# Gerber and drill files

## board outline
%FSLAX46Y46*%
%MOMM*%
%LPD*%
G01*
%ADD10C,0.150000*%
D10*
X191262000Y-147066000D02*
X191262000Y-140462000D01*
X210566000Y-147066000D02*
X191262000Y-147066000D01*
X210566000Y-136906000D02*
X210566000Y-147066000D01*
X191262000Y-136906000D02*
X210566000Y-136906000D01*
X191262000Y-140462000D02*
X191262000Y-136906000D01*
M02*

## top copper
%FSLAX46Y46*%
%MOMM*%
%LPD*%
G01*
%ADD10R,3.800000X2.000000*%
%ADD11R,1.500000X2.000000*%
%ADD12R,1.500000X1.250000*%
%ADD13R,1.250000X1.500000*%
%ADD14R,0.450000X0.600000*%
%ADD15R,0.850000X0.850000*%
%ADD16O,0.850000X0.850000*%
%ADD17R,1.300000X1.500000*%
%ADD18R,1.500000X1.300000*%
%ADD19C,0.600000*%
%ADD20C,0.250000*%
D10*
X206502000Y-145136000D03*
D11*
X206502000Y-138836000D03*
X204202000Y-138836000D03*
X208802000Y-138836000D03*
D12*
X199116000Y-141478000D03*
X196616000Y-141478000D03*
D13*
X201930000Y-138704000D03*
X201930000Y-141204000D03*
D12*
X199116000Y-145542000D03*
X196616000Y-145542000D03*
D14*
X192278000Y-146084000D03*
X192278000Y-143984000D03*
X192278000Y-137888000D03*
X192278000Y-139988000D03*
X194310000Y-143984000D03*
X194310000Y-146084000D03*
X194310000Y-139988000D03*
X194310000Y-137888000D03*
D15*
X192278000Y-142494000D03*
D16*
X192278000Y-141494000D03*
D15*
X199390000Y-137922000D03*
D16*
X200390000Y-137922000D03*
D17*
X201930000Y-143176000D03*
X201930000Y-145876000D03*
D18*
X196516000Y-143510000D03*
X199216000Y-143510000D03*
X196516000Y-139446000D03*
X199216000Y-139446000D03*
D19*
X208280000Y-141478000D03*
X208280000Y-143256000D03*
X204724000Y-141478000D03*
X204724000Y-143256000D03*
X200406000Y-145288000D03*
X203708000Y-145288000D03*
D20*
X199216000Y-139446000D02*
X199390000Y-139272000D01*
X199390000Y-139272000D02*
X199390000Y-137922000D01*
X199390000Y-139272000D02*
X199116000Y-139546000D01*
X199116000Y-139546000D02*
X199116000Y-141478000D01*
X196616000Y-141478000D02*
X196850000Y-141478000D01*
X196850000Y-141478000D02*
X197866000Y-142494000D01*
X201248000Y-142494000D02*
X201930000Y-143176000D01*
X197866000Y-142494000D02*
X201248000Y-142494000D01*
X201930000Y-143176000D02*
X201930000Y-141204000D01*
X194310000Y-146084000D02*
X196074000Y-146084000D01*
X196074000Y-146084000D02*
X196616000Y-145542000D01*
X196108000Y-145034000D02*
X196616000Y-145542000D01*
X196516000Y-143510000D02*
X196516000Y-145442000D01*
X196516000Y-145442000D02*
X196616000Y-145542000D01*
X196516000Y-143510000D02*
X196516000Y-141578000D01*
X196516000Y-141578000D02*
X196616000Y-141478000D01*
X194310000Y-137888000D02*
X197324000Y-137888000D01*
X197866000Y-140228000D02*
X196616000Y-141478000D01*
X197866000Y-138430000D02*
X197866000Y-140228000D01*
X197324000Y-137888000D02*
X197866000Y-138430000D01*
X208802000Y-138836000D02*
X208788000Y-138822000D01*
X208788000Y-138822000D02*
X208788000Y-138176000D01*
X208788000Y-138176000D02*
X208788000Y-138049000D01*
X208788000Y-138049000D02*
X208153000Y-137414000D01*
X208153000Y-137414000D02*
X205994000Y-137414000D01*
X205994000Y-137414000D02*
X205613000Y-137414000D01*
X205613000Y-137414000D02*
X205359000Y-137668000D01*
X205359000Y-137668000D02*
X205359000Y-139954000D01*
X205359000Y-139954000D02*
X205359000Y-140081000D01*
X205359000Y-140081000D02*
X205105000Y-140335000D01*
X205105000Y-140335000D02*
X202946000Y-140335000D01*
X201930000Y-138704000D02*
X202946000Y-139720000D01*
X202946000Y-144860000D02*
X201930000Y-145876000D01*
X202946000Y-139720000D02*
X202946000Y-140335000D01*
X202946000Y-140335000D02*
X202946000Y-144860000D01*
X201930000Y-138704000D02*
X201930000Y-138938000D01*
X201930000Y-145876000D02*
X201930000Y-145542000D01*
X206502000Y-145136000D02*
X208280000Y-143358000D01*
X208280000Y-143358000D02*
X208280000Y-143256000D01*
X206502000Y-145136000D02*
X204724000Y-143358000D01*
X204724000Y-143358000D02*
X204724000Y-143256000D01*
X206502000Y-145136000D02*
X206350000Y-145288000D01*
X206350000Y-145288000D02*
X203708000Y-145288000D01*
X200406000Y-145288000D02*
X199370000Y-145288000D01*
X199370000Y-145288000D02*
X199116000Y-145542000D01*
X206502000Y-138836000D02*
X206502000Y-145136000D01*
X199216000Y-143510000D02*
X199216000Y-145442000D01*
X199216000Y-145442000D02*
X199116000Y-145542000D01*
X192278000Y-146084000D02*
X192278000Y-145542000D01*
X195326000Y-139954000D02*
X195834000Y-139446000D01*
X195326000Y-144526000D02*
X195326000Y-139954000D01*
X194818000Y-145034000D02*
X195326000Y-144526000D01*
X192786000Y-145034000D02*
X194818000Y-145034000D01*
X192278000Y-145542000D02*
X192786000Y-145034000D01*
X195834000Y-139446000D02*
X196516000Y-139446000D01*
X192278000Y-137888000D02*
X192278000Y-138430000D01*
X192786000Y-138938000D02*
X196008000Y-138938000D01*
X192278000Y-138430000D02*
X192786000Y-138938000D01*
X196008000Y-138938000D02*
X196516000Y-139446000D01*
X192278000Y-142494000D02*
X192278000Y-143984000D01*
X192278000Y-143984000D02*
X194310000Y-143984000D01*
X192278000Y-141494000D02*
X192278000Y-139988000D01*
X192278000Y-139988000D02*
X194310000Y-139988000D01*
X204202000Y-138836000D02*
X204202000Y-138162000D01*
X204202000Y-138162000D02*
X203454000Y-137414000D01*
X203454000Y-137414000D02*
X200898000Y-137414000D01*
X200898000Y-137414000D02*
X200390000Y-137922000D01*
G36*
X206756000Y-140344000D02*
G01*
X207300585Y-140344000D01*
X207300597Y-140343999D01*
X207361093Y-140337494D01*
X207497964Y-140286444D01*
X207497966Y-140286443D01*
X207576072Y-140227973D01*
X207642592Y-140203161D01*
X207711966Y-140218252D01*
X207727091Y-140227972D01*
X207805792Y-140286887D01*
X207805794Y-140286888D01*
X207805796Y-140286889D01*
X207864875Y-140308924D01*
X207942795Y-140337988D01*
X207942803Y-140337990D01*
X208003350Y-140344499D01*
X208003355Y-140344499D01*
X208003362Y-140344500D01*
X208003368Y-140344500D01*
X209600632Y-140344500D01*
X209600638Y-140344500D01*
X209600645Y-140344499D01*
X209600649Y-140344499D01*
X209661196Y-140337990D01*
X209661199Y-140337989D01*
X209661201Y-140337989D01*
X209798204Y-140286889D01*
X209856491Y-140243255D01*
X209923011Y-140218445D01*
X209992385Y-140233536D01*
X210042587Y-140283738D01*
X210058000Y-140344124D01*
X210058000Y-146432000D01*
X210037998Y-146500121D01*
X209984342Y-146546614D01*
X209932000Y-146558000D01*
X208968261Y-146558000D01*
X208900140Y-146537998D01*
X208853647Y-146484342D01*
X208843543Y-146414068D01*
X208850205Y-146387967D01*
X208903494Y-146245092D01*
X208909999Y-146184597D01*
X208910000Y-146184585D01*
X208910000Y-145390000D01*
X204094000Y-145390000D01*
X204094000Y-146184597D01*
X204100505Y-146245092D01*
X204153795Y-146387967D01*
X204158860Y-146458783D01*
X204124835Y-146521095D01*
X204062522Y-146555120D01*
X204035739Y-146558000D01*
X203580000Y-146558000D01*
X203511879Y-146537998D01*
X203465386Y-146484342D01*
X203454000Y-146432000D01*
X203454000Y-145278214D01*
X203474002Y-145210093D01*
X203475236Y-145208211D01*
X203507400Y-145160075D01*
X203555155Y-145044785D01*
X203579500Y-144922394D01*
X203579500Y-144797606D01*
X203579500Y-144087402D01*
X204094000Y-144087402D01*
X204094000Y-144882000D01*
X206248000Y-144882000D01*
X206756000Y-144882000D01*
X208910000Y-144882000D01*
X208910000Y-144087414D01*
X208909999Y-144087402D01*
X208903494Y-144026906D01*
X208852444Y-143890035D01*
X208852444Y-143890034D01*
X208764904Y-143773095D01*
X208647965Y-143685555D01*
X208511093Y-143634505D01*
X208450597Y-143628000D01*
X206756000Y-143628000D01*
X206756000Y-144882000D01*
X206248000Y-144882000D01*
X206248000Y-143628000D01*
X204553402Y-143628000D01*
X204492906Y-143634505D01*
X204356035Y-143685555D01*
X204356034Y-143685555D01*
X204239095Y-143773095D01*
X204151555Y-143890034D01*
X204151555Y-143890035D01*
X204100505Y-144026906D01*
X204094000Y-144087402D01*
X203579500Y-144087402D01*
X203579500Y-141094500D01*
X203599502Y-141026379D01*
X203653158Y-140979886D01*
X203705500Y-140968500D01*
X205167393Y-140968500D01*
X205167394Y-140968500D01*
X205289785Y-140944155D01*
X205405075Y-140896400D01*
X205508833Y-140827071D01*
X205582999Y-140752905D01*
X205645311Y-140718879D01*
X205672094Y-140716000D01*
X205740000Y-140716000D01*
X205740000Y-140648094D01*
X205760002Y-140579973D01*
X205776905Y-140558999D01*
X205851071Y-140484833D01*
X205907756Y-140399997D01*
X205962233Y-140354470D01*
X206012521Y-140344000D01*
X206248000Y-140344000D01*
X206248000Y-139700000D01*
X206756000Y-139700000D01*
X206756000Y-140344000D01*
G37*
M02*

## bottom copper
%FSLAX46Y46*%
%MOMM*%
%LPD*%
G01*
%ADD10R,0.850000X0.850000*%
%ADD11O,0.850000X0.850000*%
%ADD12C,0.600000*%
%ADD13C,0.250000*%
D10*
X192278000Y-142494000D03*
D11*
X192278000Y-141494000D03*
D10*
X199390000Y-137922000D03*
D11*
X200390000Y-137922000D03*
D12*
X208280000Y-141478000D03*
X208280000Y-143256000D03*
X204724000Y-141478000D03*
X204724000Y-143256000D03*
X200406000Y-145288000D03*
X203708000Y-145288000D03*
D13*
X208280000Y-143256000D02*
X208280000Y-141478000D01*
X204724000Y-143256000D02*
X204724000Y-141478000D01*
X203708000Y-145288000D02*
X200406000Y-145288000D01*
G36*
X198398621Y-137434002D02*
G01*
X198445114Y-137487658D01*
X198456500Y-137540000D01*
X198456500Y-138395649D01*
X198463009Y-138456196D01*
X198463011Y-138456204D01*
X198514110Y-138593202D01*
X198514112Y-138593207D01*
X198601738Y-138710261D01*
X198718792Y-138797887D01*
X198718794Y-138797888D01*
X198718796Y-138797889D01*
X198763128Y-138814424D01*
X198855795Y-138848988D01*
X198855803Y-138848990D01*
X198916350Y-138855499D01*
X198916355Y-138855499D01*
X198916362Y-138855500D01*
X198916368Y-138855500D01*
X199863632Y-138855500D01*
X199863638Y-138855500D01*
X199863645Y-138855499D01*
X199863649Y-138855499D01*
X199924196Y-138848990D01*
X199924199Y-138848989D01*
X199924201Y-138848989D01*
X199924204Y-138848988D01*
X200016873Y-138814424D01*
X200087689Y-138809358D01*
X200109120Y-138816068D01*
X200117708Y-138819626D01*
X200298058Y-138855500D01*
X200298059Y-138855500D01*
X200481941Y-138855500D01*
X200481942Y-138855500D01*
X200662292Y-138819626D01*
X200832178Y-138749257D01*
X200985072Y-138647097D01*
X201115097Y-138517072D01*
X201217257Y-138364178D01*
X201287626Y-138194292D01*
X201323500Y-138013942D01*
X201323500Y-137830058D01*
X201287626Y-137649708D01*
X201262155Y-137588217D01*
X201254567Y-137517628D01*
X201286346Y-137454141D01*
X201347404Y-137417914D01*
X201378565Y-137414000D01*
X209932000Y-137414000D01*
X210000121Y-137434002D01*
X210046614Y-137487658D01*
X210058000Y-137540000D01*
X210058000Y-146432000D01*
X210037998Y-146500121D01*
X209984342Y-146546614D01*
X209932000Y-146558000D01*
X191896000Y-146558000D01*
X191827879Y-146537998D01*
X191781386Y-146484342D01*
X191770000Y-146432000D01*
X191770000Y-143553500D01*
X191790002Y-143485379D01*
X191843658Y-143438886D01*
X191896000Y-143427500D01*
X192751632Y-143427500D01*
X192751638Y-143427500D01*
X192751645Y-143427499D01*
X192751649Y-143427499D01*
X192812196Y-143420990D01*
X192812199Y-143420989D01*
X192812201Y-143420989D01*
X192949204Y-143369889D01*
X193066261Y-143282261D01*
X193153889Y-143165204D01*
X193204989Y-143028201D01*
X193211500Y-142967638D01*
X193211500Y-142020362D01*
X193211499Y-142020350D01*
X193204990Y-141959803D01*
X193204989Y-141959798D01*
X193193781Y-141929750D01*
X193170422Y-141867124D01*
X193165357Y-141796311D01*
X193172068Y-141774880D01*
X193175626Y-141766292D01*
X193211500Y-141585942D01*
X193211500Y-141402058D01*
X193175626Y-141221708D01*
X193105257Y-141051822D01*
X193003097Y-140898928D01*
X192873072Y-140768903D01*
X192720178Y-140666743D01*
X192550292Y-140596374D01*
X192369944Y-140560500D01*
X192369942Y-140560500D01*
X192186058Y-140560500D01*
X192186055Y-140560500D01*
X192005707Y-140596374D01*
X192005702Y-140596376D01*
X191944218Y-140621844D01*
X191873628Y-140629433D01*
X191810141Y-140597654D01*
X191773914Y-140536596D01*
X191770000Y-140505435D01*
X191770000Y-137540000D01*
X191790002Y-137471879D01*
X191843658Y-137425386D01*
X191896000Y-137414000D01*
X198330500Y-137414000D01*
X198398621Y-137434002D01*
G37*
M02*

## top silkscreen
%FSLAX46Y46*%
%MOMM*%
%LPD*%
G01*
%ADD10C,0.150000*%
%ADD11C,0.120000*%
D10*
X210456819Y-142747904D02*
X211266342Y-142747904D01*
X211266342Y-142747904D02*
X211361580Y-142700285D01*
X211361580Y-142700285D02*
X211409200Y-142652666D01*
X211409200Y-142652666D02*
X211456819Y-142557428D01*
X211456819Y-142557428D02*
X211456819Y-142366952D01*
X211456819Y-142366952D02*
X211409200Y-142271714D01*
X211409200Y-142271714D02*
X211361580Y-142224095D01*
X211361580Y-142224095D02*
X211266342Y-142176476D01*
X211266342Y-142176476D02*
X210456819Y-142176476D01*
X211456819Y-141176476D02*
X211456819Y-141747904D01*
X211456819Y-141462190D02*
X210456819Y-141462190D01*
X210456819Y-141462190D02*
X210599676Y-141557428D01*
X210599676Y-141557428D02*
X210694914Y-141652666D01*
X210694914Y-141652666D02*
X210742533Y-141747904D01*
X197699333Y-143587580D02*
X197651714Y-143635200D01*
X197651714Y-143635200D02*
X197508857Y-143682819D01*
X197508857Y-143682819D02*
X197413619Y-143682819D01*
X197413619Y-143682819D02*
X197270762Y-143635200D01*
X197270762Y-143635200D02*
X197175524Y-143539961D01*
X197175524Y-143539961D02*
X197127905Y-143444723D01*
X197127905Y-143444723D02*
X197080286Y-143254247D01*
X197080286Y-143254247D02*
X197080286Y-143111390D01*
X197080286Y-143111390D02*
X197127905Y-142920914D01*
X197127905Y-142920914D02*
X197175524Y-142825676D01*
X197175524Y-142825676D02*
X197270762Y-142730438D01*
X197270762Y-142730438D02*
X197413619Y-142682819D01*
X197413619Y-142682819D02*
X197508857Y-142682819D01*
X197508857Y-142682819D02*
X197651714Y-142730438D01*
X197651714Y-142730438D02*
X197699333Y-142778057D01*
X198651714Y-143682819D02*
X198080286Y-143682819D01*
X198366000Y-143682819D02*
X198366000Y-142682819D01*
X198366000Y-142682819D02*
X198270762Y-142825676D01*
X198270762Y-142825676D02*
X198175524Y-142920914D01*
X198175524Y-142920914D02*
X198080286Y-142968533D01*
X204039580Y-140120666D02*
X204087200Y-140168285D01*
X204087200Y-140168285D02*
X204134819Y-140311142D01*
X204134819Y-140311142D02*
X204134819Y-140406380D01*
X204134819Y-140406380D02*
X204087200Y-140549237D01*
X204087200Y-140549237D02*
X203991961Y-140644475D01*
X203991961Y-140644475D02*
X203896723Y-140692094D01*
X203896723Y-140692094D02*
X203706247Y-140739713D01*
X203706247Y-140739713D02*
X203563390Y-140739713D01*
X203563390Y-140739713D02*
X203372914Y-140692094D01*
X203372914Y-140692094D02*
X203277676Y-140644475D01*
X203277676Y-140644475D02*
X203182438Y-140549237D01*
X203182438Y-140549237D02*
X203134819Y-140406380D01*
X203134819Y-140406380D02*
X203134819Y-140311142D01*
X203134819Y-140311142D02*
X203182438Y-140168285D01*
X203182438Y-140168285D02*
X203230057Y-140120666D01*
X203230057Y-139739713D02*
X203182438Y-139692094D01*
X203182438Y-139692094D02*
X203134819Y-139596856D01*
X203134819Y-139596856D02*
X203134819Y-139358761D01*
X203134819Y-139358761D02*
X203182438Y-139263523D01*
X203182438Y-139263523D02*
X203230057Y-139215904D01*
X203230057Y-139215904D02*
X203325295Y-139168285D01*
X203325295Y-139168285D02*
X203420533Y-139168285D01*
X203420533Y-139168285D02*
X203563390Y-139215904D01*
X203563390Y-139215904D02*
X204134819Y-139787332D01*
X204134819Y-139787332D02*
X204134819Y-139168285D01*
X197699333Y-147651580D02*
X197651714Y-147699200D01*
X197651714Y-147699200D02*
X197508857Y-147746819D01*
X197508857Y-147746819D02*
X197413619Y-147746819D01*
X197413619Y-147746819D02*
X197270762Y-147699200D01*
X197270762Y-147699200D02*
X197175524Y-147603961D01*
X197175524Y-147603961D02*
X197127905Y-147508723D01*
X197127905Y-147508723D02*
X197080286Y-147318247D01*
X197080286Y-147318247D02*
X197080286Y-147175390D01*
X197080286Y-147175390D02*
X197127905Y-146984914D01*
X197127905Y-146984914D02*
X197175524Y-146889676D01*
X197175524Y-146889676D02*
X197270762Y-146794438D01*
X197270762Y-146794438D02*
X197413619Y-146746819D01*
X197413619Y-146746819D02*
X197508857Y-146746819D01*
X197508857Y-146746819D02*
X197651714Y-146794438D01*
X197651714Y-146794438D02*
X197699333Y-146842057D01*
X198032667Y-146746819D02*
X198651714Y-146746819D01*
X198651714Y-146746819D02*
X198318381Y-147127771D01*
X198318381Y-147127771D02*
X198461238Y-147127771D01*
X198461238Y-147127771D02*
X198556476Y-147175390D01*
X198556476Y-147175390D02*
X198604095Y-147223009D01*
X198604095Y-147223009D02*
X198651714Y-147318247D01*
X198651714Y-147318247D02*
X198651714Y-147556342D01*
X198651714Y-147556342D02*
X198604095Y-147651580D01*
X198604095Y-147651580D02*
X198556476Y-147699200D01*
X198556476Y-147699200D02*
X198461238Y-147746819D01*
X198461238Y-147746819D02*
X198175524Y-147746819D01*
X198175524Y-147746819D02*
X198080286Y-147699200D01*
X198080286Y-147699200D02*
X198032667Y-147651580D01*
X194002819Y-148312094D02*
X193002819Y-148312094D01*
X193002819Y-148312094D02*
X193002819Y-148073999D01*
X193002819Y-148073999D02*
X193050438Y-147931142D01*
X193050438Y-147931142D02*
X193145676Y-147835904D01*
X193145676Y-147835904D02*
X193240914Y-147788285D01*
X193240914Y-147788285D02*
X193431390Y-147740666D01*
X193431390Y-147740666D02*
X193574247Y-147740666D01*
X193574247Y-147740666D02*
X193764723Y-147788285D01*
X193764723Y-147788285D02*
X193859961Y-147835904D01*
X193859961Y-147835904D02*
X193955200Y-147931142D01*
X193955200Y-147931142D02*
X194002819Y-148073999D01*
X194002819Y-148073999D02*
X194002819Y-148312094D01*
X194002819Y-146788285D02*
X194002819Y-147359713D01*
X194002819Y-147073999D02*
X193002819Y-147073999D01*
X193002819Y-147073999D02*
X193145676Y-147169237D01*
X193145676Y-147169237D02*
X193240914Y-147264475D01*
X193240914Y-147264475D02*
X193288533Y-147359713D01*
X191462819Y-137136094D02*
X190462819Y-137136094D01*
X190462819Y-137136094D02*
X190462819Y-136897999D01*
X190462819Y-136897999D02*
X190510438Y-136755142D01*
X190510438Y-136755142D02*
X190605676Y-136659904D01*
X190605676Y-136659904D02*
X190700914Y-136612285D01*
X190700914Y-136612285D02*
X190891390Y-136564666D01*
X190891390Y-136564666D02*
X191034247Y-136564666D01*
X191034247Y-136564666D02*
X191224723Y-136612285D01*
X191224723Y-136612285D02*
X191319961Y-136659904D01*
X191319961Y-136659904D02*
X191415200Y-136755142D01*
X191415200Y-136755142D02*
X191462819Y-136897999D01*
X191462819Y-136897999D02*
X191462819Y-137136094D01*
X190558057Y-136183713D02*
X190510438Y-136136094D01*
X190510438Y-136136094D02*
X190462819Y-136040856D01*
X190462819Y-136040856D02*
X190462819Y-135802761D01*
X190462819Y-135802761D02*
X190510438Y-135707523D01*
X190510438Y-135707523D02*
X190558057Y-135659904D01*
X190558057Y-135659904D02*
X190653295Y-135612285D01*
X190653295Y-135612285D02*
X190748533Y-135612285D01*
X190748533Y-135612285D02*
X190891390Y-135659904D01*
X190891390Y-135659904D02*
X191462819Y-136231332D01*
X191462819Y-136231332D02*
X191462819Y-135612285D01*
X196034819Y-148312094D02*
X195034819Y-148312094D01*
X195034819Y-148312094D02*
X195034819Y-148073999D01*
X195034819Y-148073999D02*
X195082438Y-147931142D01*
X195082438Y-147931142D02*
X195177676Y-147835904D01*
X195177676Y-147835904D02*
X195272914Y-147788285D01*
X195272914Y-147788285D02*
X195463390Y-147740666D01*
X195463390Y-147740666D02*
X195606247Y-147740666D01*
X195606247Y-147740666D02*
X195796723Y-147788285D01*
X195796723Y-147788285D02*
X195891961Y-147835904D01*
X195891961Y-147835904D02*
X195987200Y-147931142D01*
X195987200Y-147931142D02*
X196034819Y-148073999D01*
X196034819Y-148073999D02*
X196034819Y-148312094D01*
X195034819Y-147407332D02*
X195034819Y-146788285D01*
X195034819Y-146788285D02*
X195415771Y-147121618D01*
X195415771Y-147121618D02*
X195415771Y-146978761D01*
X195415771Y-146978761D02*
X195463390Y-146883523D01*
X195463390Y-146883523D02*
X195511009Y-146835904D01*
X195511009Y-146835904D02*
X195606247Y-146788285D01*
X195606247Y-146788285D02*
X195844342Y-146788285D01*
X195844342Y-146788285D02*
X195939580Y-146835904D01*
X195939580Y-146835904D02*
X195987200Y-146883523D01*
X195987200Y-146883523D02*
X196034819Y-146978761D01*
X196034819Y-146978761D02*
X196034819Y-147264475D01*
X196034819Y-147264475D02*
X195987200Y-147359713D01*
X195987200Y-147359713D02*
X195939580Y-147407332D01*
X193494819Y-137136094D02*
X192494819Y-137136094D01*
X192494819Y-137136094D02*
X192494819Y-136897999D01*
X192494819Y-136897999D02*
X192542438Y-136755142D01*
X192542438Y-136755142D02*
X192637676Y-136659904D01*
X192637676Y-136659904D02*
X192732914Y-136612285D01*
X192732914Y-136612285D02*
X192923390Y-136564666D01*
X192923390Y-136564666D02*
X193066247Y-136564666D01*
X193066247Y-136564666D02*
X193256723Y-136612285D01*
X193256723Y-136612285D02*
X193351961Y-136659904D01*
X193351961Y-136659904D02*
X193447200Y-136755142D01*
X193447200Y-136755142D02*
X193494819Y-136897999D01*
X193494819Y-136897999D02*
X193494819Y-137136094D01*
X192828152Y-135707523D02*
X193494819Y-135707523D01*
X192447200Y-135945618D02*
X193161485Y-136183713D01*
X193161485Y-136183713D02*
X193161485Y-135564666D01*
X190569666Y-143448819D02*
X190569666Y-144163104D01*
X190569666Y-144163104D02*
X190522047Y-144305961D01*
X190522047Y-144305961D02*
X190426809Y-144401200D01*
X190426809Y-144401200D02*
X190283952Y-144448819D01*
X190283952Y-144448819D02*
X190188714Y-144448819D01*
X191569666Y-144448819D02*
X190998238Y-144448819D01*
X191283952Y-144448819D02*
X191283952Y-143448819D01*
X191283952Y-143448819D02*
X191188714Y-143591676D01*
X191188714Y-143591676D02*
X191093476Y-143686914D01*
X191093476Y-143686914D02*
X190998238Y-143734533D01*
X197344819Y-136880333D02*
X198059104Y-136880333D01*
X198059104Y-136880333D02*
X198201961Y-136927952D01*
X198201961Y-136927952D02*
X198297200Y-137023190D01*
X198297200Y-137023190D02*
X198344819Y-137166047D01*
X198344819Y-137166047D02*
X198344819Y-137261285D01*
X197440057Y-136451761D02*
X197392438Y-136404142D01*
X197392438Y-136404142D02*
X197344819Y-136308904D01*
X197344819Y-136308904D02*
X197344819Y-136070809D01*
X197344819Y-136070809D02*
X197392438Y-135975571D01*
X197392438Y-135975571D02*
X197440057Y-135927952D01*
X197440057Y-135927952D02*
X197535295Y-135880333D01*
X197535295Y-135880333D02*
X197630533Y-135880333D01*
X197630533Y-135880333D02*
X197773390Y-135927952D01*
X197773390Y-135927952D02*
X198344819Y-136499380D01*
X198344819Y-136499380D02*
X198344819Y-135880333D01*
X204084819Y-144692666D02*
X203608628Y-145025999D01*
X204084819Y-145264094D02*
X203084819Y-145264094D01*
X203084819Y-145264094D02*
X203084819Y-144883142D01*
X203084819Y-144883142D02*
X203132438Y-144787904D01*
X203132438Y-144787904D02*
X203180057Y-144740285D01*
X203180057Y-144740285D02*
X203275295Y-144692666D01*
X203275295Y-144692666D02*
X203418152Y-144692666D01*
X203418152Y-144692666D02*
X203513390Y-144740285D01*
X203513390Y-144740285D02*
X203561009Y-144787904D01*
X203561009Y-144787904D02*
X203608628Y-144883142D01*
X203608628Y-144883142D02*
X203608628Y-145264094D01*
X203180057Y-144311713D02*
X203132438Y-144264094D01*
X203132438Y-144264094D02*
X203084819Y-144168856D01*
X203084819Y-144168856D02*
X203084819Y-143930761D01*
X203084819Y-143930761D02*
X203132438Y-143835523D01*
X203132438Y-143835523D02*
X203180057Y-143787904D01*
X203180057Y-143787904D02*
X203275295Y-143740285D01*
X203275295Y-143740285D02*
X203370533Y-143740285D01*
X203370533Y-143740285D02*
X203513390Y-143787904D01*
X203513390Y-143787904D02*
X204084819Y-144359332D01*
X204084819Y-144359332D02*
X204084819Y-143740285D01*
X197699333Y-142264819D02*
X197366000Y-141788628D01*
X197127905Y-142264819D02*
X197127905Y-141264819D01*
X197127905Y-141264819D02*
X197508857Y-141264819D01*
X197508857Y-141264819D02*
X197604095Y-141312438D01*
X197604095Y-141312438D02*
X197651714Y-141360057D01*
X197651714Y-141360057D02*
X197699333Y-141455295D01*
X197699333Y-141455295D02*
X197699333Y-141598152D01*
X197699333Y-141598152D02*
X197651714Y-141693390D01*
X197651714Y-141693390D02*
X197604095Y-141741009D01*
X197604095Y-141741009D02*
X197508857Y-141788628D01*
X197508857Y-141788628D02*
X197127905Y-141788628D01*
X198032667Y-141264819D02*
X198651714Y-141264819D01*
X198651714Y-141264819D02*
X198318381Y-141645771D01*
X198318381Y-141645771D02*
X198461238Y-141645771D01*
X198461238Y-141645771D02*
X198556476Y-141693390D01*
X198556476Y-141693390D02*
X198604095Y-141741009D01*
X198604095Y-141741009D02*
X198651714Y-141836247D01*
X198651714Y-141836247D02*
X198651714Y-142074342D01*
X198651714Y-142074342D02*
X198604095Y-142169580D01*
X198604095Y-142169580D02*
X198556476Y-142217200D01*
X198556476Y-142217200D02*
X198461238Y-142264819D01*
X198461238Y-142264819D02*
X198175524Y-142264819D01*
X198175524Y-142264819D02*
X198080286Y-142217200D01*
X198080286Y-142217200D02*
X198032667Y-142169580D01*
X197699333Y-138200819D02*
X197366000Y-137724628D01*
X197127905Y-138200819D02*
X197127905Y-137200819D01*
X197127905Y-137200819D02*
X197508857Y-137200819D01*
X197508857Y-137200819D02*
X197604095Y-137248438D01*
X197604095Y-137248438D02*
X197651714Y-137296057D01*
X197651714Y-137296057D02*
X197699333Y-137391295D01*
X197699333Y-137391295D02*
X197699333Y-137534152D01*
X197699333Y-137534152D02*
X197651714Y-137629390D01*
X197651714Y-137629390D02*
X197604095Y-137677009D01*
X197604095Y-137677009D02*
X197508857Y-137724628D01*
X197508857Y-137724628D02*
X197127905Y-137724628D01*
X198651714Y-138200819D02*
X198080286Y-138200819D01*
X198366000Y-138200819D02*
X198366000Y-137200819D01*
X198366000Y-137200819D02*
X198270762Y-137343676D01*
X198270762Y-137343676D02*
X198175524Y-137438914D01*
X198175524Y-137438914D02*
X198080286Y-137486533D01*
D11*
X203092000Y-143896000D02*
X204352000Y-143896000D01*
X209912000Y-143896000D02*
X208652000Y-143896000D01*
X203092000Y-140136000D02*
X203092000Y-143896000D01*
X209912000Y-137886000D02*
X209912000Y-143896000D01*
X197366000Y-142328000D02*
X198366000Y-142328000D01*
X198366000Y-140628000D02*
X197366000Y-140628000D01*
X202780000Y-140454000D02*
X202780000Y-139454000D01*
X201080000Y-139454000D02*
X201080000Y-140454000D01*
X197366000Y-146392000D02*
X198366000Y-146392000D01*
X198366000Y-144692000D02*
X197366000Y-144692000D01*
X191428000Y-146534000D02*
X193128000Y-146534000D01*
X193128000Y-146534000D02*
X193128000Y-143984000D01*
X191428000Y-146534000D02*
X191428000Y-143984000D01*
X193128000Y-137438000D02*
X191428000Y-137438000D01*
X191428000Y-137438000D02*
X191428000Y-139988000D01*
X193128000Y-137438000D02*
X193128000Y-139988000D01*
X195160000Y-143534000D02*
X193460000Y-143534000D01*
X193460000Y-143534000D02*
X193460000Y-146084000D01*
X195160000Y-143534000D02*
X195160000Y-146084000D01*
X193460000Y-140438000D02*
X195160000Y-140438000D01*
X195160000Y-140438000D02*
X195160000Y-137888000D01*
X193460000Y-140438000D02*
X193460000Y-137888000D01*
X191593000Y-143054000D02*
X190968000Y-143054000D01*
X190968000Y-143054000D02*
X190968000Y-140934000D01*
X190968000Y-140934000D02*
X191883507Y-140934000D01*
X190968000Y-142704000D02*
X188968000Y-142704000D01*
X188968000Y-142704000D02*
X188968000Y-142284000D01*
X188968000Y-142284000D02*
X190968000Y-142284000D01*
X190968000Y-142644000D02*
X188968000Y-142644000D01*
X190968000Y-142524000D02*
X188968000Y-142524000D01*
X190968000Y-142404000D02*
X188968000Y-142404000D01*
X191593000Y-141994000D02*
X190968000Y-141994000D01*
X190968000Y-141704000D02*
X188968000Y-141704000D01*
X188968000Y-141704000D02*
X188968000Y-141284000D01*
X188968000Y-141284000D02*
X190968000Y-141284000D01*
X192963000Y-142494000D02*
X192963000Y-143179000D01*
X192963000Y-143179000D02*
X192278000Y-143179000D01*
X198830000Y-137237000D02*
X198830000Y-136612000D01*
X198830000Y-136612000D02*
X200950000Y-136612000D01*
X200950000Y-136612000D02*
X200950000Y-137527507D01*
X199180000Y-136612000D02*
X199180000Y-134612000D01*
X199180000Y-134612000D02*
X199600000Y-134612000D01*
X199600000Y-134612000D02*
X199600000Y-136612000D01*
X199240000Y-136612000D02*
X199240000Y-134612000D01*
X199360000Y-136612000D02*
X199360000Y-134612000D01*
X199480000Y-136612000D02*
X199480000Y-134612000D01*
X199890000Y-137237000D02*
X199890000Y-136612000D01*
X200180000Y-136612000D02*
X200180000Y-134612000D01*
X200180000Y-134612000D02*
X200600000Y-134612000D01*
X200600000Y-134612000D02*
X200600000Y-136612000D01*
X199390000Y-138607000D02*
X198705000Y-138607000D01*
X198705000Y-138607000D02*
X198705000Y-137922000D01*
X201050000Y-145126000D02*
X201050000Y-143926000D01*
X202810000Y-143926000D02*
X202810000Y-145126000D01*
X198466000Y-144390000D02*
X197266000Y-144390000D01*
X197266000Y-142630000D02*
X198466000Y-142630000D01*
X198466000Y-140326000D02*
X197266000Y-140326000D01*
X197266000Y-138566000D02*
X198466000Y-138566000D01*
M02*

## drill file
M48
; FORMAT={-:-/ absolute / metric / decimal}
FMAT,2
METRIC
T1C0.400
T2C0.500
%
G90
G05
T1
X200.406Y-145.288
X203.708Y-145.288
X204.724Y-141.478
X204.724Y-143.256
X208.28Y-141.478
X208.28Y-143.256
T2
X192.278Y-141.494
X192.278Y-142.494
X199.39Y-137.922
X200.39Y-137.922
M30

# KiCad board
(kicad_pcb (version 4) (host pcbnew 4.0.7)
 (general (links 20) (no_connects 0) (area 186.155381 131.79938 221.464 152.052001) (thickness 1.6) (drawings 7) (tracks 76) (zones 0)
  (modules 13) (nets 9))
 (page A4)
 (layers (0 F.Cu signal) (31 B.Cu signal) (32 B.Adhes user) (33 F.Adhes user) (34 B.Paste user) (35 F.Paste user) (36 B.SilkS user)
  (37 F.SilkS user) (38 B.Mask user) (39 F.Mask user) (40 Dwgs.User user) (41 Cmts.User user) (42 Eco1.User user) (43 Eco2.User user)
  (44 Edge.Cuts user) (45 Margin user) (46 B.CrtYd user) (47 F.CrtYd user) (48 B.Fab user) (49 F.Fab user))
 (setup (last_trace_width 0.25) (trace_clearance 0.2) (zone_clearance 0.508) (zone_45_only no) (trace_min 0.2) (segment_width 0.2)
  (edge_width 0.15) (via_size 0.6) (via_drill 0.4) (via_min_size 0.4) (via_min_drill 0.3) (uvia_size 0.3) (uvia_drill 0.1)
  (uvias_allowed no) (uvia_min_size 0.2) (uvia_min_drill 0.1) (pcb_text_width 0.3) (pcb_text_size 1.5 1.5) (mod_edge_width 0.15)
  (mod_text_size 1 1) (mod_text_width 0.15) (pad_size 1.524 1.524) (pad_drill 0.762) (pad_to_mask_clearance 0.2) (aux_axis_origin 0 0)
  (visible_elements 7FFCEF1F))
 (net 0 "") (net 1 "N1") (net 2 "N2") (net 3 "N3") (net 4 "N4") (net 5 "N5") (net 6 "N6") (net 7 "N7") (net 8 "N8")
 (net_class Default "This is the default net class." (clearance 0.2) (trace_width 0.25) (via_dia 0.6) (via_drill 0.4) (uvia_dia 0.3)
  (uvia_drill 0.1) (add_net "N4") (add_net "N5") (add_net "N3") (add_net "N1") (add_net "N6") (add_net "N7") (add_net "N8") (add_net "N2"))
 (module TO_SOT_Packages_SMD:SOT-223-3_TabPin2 (layer F.Cu) (at 206.502 141.986 270)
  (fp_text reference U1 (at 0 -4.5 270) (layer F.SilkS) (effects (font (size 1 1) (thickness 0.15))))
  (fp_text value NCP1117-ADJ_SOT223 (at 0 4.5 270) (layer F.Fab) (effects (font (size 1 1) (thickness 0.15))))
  (fp_line (start 1.91 3.41) (end 1.91 2.15) (layer F.SilkS) (width 0.12))
  (fp_line (start 1.91 -3.41) (end 1.91 -2.15) (layer F.SilkS) (width 0.12))
  (fp_line (start -1.85 3.41) (end 1.91 3.41) (layer F.SilkS) (width 0.12))
  (fp_line (start -4.1 -3.41) (end 1.91 -3.41) (layer F.SilkS) (width 0.12))
  (pad 2 smd rect (at 3.15 0 270) (size 2 3.8) (layers F.Cu F.Paste F.Mask) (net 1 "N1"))
  (pad 2 smd rect (at -3.15 0 270) (size 2 1.5) (layers F.Cu F.Paste F.Mask) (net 1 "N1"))
  (pad 3 smd rect (at -3.15 2.3 270) (size 2 1.5) (layers F.Cu F.Paste F.Mask) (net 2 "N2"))
  (pad 1 smd rect (at -3.15 -2.3 270) (size 2 1.5) (layers F.Cu F.Paste F.Mask) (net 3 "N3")))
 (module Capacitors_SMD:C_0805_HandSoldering (layer F.Cu) (at 197.866 141.478 180)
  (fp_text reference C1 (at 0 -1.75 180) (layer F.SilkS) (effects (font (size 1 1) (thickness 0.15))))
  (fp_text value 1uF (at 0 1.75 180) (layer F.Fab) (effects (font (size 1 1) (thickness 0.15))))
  (fp_line (start 0.5 -0.85) (end -0.5 -0.85) (layer F.SilkS) (width 0.12))
  (fp_line (start -0.5 0.85) (end 0.5 0.85) (layer F.SilkS) (width 0.12))
  (pad 1 smd rect (at -1.25 0 180) (size 1.5 1.25) (layers F.Cu F.Paste F.Mask) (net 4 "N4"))
  (pad 2 smd rect (at 1.25 0 180) (size 1.5 1.25) (layers F.Cu F.Paste F.Mask) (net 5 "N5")))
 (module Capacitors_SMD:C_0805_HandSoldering (layer F.Cu) (at 201.93 139.954 270)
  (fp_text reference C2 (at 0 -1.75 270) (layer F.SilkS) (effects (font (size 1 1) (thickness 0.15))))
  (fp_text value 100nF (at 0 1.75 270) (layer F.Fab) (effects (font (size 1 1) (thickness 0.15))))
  (fp_line (start 0.5 -0.85) (end -0.5 -0.85) (layer F.SilkS) (width 0.12))
  (fp_line (start -0.5 0.85) (end 0.5 0.85) (layer F.SilkS) (width 0.12))
  (pad 1 smd rect (at -1.25 0 270) (size 1.5 1.25) (layers F.Cu F.Paste F.Mask) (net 3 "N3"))
  (pad 2 smd rect (at 1.25 0 270) (size 1.5 1.25) (layers F.Cu F.Paste F.Mask) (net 5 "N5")))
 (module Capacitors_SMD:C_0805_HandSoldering (layer F.Cu) (at 197.866 145.542 180)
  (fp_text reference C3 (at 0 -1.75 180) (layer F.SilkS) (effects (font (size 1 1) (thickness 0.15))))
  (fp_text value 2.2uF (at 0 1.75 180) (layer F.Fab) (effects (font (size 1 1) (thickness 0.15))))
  (fp_line (start 0.5 -0.85) (end -0.5 -0.85) (layer F.SilkS) (width 0.12))
  (fp_line (start -0.5 0.85) (end 0.5 0.85) (layer F.SilkS) (width 0.12))
  (pad 1 smd rect (at -1.25 0 180) (size 1.5 1.25) (layers F.Cu F.Paste F.Mask) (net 1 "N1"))
  (pad 2 smd rect (at 1.25 0 180) (size 1.5 1.25) (layers F.Cu F.Paste F.Mask) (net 5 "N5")))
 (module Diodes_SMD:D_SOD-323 (layer F.Cu) (at 192.278 145.034 90)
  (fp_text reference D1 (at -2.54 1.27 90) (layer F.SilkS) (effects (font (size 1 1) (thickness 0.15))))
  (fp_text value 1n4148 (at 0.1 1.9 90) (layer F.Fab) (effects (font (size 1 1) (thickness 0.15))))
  (fp_line (start -1.5 -0.85) (end -1.5 0.85) (layer F.SilkS) (width 0.12))
  (fp_line (start -1.5 0.85) (end 1.05 0.85) (layer F.SilkS) (width 0.12))
  (fp_line (start -1.5 -0.85) (end 1.05 -0.85) (layer F.SilkS) (width 0.12))
  (pad 1 smd rect (at -1.05 0 90) (size 0.6 0.45) (layers F.Cu F.Paste F.Mask) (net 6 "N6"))
  (pad 2 smd rect (at 1.05 0 90) (size 0.6 0.45) (layers F.Cu F.Paste F.Mask) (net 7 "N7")))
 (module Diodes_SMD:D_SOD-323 (layer F.Cu) (at 192.278 138.938 270)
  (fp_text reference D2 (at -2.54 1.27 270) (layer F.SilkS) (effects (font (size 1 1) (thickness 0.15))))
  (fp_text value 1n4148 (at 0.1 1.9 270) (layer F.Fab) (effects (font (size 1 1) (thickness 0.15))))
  (fp_line (start -1.5 -0.85) (end -1.5 0.85) (layer F.SilkS) (width 0.12))
  (fp_line (start -1.5 0.85) (end 1.05 0.85) (layer F.SilkS) (width 0.12))
  (fp_line (start -1.5 -0.85) (end 1.05 -0.85) (layer F.SilkS) (width 0.12))
  (pad 1 smd rect (at -1.05 0 270) (size 0.6 0.45) (layers F.Cu F.Paste F.Mask) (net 6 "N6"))
  (pad 2 smd rect (at 1.05 0 270) (size 0.6 0.45) (layers F.Cu F.Paste F.Mask) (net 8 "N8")))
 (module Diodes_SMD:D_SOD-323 (layer F.Cu) (at 194.31 145.034 270)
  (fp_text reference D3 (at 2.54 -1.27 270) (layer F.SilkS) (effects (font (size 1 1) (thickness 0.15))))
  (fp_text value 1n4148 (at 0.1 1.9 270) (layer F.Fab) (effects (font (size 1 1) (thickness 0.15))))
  (fp_line (start -1.5 -0.85) (end -1.5 0.85) (layer F.SilkS) (width 0.12))
  (fp_line (start -1.5 0.85) (end 1.05 0.85) (layer F.SilkS) (width 0.12))
  (fp_line (start -1.5 -0.85) (end 1.05 -0.85) (layer F.SilkS) (width 0.12))
  (pad 1 smd rect (at -1.05 0 270) (size 0.6 0.45) (layers F.Cu F.Paste F.Mask) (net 7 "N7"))
  (pad 2 smd rect (at 1.05 0 270) (size 0.6 0.45) (layers F.Cu F.Paste F.Mask) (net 5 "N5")))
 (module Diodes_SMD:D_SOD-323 (layer F.Cu) (at 194.31 138.938 90)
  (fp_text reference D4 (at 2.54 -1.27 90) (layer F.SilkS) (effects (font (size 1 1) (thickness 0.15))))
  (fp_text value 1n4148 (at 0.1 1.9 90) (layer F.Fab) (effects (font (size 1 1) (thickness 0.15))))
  (fp_line (start -1.5 -0.85) (end -1.5 0.85) (layer F.SilkS) (width 0.12))
  (fp_line (start -1.5 0.85) (end 1.05 0.85) (layer F.SilkS) (width 0.12))
  (fp_line (start -1.5 -0.85) (end 1.05 -0.85) (layer F.SilkS) (width 0.12))
  (pad 1 smd rect (at -1.05 0 90) (size 0.6 0.45) (layers F.Cu F.Paste F.Mask) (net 8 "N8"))
  (pad 2 smd rect (at 1.05 0 90) (size 0.6 0.45) (layers F.Cu F.Paste F.Mask) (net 5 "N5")))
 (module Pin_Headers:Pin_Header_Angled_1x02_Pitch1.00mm (layer F.Cu) (at 192.278 142.494 180)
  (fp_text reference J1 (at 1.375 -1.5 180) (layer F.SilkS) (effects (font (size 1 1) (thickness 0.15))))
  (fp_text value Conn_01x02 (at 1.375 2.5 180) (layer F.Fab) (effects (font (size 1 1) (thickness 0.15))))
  (fp_line (start 0.685 -0.56) (end 1.31 -0.56) (layer F.SilkS) (width 0.12))
  (fp_line (start 1.31 -0.56) (end 1.31 1.56) (layer F.SilkS) (width 0.12))
  (fp_line (start 1.31 1.56) (end 0.394493 1.56) (layer F.SilkS) (width 0.12))
  (fp_line (start 1.31 -0.21) (end 3.31 -0.21) (layer F.SilkS) (width 0.12))
  (fp_line (start 3.31 -0.21) (end 3.31 0.21) (layer F.SilkS) (width 0.12))
  (fp_line (start 3.31 0.21) (end 1.31 0.21) (layer F.SilkS) (width 0.12))
  (fp_line (start 1.31 -0.15) (end 3.31 -0.15) (layer F.SilkS) (width 0.12))
  (fp_line (start 1.31 -0.03) (end 3.31 -0.03) (layer F.SilkS) (width 0.12))
  (fp_line (start 1.31 0.09) (end 3.31 0.09) (layer F.SilkS) (width 0.12))
  (fp_line (start 0.685 0.5) (end 1.31 0.5) (layer F.SilkS) (width 0.12))
  (fp_line (start 1.31 0.79) (end 3.31 0.79) (layer F.SilkS) (width 0.12))
  (fp_line (start 3.31 0.79) (end 3.31 1.21) (layer F.SilkS) (width 0.12))
  (fp_line (start 3.31 1.21) (end 1.31 1.21) (layer F.SilkS) (width 0.12))
  (fp_line (start -0.685 0) (end -0.685 -0.685) (layer F.SilkS) (width 0.12))
  (fp_line (start -0.685 -0.685) (end 0 -0.685) (layer F.SilkS) (width 0.12))
  (pad 1 thru_hole rect (at 0 0 180) (size 0.85 0.85) (drill 0.5) (layers *.Cu *.Mask) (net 7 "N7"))
  (pad 2 thru_hole oval (at 0 1 180) (size 0.85 0.85) (drill 0.5) (layers *.Cu *.Mask) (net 8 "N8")))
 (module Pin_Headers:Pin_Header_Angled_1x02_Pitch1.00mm (layer F.Cu) (at 199.39 137.922 90)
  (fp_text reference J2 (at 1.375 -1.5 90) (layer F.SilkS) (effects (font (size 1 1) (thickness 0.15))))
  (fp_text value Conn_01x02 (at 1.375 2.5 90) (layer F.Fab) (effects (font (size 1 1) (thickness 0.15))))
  (fp_line (start 0.685 -0.56) (end 1.31 -0.56) (layer F.SilkS) (width 0.12))
  (fp_line (start 1.31 -0.56) (end 1.31 1.56) (layer F.SilkS) (width 0.12))
  (fp_line (start 1.31 1.56) (end 0.394493 1.56) (layer F.SilkS) (width 0.12))
  (fp_line (start 1.31 -0.21) (end 3.31 -0.21) (layer F.SilkS) (width 0.12))
  (fp_line (start 3.31 -0.21) (end 3.31 0.21) (layer F.SilkS) (width 0.12))
  (fp_line (start 3.31 0.21) (end 1.31 0.21) (layer F.SilkS) (width 0.12))
  (fp_line (start 1.31 -0.15) (end 3.31 -0.15) (layer F.SilkS) (width 0.12))
  (fp_line (start 1.31 -0.03) (end 3.31 -0.03) (layer F.SilkS) (width 0.12))
  (fp_line (start 1.31 0.09) (end 3.31 0.09) (layer F.SilkS) (width 0.12))
  (fp_line (start 0.685 0.5) (end 1.31 0.5) (layer F.SilkS) (width 0.12))
  (fp_line (start 1.31 0.79) (end 3.31 0.79) (layer F.SilkS) (width 0.12))
  (fp_line (start 3.31 0.79) (end 3.31 1.21) (layer F.SilkS) (width 0.12))
  (fp_line (start 3.31 1.21) (end 1.31 1.21) (layer F.SilkS) (width 0.12))
  (fp_line (start -0.685 0) (end -0.685 -0.685) (layer F.SilkS) (width 0.12))
  (fp_line (start -0.685 -0.685) (end 0 -0.685) (layer F.SilkS) (width 0.12))
  (pad 1 thru_hole rect (at 0 0 90) (size 0.85 0.85) (drill 0.5) (layers *.Cu *.Mask) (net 4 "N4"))
  (pad 2 thru_hole oval (at 0 1 90) (size 0.85 0.85) (drill 0.5) (layers *.Cu *.Mask) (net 2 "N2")))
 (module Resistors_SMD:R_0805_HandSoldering (layer F.Cu) (at 201.93 144.526 270)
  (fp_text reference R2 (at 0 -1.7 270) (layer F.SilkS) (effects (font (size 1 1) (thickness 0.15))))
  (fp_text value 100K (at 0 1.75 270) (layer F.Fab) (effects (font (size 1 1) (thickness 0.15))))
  (fp_line (start 0.6 0.88) (end -0.6 0.88) (layer F.SilkS) (width 0.12))
  (fp_line (start -0.6 -0.88) (end 0.6 -0.88) (layer F.SilkS) (width 0.12))
  (pad 1 smd rect (at -1.35 0 270) (size 1.5 1.3) (layers F.Cu F.Paste F.Mask) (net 5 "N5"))
  (pad 2 smd rect (at 1.35 0 270) (size 1.5 1.3) (layers F.Cu F.Paste F.Mask) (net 3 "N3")))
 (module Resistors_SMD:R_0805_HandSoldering (layer F.Cu) (at 197.866 143.51)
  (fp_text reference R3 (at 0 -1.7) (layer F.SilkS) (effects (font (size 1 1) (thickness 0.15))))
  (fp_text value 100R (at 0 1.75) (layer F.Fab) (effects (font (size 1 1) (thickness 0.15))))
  (fp_line (start 0.6 0.88) (end -0.6 0.88) (layer F.SilkS) (width 0.12))
  (fp_line (start -0.6 -0.88) (end 0.6 -0.88) (layer F.SilkS) (width 0.12))
  (pad 1 smd rect (at -1.35 0) (size 1.5 1.3) (layers F.Cu F.Paste F.Mask) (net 5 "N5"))
  (pad 2 smd rect (at 1.35 0) (size 1.5 1.3) (layers F.Cu F.Paste F.Mask) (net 1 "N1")))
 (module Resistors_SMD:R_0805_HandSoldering (layer F.Cu) (at 197.866 139.446)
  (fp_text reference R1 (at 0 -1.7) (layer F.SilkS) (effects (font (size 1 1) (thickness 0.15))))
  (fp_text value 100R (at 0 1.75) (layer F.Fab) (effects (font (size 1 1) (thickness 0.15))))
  (fp_line (start 0.6 0.88) (end -0.6 0.88) (layer F.SilkS) (width 0.12))
  (fp_line (start -0.6 -0.88) (end 0.6 -0.88) (layer F.SilkS) (width 0.12))
  (pad 1 smd rect (at -1.35 0) (size 1.5 1.3) (layers F.Cu F.Paste F.Mask) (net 6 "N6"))
  (pad 2 smd rect (at 1.35 0) (size 1.5 1.3) (layers F.Cu F.Paste F.Mask) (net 4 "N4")))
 (gr_line (start 191.262 147.066) (end 191.262 140.462) (angle 90) (layer Edge.Cuts) (width 0.15))
 (gr_line (start 210.566 147.066) (end 191.262 147.066) (angle 90) (layer Edge.Cuts) (width 0.15))
 (gr_line (start 210.566 136.906) (end 210.566 147.066) (angle 90) (layer Edge.Cuts) (width 0.15))
 (gr_line (start 191.262 136.906) (end 210.566 136.906) (angle 90) (layer Edge.Cuts) (width 0.15))
 (gr_line (start 191.262 140.462) (end 191.262 136.906) (angle 90) (layer Edge.Cuts) (width 0.15))
 (segment (start 199.216 139.446) (end 199.39 139.272) (width 0.25) (layer F.Cu) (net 4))
 (segment (start 199.39 139.272) (end 199.39 137.922) (width 0.25) (layer F.Cu) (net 4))
 (segment (start 199.39 139.272) (end 199.116 139.546) (width 0.25) (layer F.Cu) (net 4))
 (segment (start 199.116 139.546) (end 199.116 141.478) (width 0.25) (layer F.Cu) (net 4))
 (segment (start 196.616 141.478) (end 196.85 141.478) (width 0.25) (layer F.Cu) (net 5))
 (segment (start 196.85 141.478) (end 197.866 142.494) (width 0.25) (layer F.Cu) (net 5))
 (segment (start 201.248 142.494) (end 201.93 143.176) (width 0.25) (layer F.Cu) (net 5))
 (segment (start 197.866 142.494) (end 201.248 142.494) (width 0.25) (layer F.Cu) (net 5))
 (segment (start 201.93 143.176) (end 201.93 141.204) (width 0.25) (layer F.Cu) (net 5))
 (segment (start 194.31 146.084) (end 196.074 146.084) (width 0.25) (layer F.Cu) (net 5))
 (segment (start 196.074 146.084) (end 196.616 145.542) (width 0.25) (layer F.Cu) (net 5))
 (segment (start 196.108 145.034) (end 196.616 145.542) (width 0.25) (layer F.Cu) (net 5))
 (segment (start 196.516 143.51) (end 196.516 145.442) (width 0.25) (layer F.Cu) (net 5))
 (segment (start 196.516 145.442) (end 196.616 145.542) (width 0.25) (layer F.Cu) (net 5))
 (segment (start 196.516 143.51) (end 196.516 141.578) (width 0.25) (layer F.Cu) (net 5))
 (segment (start 196.516 141.578) (end 196.616 141.478) (width 0.25) (layer F.Cu) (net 5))
 (segment (start 194.31 137.888) (end 197.324 137.888) (width 0.25) (layer F.Cu) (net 5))
 (segment (start 197.866 140.228) (end 196.616 141.478) (width 0.25) (layer F.Cu) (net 5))
 (segment (start 197.866 138.43) (end 197.866 140.228) (width 0.25) (layer F.Cu) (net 5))
 (segment (start 197.324 137.888) (end 197.866 138.43) (width 0.25) (layer F.Cu) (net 5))
 (segment (start 208.802 138.836) (end 208.788 138.822) (width 0.25) (layer F.Cu) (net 3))
 (segment (start 208.788 138.822) (end 208.788 138.176) (width 0.25) (layer F.Cu) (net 3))
 (segment (start 208.788 138.176) (end 208.788 138.049) (width 0.25) (layer F.Cu) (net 3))
 (segment (start 208.788 138.049) (end 208.153 137.414) (width 0.25) (layer F.Cu) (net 3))
 (segment (start 208.153 137.414) (end 205.994 137.414) (width 0.25) (layer F.Cu) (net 3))
 (segment (start 205.994 137.414) (end 205.613 137.414) (width 0.25) (layer F.Cu) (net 3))
 (segment (start 205.613 137.414) (end 205.359 137.668) (width 0.25) (layer F.Cu) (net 3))
 (segment (start 205.359 137.668) (end 205.359 139.954) (width 0.25) (layer F.Cu) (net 3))
 (segment (start 205.359 139.954) (end 205.359 140.081) (width 0.25) (layer F.Cu) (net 3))
 (segment (start 205.359 140.081) (end 205.105 140.335) (width 0.25) (layer F.Cu) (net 3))
 (segment (start 205.105 140.335) (end 202.946 140.335) (width 0.25) (layer F.Cu) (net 3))
 (segment (start 201.93 138.704) (end 202.946 139.72) (width 0.25) (layer F.Cu) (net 3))
 (segment (start 202.946 144.86) (end 201.93 145.876) (width 0.25) (layer F.Cu) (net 3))
 (segment (start 202.946 139.72) (end 202.946 140.335) (width 0.25) (layer F.Cu) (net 3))
 (segment (start 202.946 140.335) (end 202.946 144.86) (width 0.25) (layer F.Cu) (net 3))
 (segment (start 201.93 138.704) (end 201.93 138.938) (width 0.25) (layer F.Cu) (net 3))
 (segment (start 201.93 145.876) (end 201.93 145.542) (width 0.25) (layer F.Cu) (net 3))
 (segment (start 206.502 145.136) (end 208.28 143.358) (width 0.25) (layer F.Cu) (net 1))
 (via (at 208.28 141.478) (size 0.6) (drill 0.4) (layers F.Cu B.Cu) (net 1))
 (segment (start 208.28 143.256) (end 208.28 141.478) (width 0.25) (layer B.Cu) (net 1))
 (via (at 208.28 143.256) (size 0.6) (drill 0.4) (layers F.Cu B.Cu) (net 1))
 (segment (start 208.28 143.358) (end 208.28 143.256) (width 0.25) (layer F.Cu) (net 1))
 (segment (start 206.502 145.136) (end 204.724 143.358) (width 0.25) (layer F.Cu) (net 1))
 (via (at 204.724 141.478) (size 0.6) (drill 0.4) (layers F.Cu B.Cu) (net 1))
 (segment (start 204.724 143.256) (end 204.724 141.478) (width 0.25) (layer B.Cu) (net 1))
 (via (at 204.724 143.256) (size 0.6) (drill 0.4) (layers F.Cu B.Cu) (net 1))
 (segment (start 204.724 143.358) (end 204.724 143.256) (width 0.25) (layer F.Cu) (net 1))
 (segment (start 206.502 145.136) (end 206.35 145.288) (width 0.25) (layer F.Cu) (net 1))
 (segment (start 206.35 145.288) (end 203.708 145.288) (width 0.25) (layer F.Cu) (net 1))
 (segment (start 200.406 145.288) (end 199.37 145.288) (width 0.25) (layer F.Cu) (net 1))
 (via (at 200.406 145.288) (size 0.6) (drill 0.4) (layers F.Cu B.Cu) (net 1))
 (segment (start 203.708 145.288) (end 200.406 145.288) (width 0.25) (layer B.Cu) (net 1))
 (via (at 203.708 145.288) (size 0.6) (drill 0.4) (layers F.Cu B.Cu) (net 1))
 (segment (start 199.37 145.288) (end 199.116 145.542) (width 0.25) (layer F.Cu) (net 1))
 (segment (start 206.502 138.836) (end 206.502 145.136) (width 0.25) (layer F.Cu) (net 1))
 (segment (start 199.216 143.51) (end 199.216 145.442) (width 0.25) (layer F.Cu) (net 1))
 (segment (start 199.216 145.442) (end 199.116 145.542) (width 0.25) (layer F.Cu) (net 1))
 (segment (start 192.278 146.084) (end 192.278 145.542) (width 0.25) (layer F.Cu) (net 6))
 (segment (start 195.326 139.954) (end 195.834 139.446) (width 0.25) (layer F.Cu) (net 6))
 (segment (start 195.326 144.526) (end 195.326 139.954) (width 0.25) (layer F.Cu) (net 6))
 (segment (start 194.818 145.034) (end 195.326 144.526) (width 0.25) (layer F.Cu) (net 6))
 (segment (start 192.786 145.034) (end 194.818 145.034) (width 0.25) (layer F.Cu) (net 6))
 (segment (start 192.278 145.542) (end 192.786 145.034) (width 0.25) (layer F.Cu) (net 6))
 (segment (start 195.834 139.446) (end 196.516 139.446) (width 0.25) (layer F.Cu) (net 6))
 (segment (start 192.278 137.888) (end 192.278 138.43) (width 0.25) (layer F.Cu) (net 6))
 (segment (start 192.786 138.938) (end 196.008 138.938) (width 0.25) (layer F.Cu) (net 6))
 (segment (start 192.278 138.43) (end 192.786 138.938) (width 0.25) (layer F.Cu) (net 6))
 (segment (start 196.008 138.938) (end 196.516 139.446) (width 0.25) (layer F.Cu) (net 6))
 (segment (start 192.278 142.494) (end 192.278 143.984) (width 0.25) (layer F.Cu) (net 7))
 (segment (start 192.278 143.984) (end 194.31 143.984) (width 0.25) (layer F.Cu) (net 7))
 (segment (start 192.278 141.494) (end 192.278 139.988) (width 0.25) (layer F.Cu) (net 8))
 (segment (start 192.278 139.988) (end 194.31 139.988) (width 0.25) (layer F.Cu) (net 8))
 (segment (start 204.202 138.836) (end 204.202 138.162) (width 0.25) (layer F.Cu) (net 2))
 (segment (start 204.202 138.162) (end 203.454 137.414) (width 0.25) (layer F.Cu) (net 2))
 (segment (start 203.454 137.414) (end 200.898 137.414) (width 0.25) (layer F.Cu) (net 2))
 (segment (start 200.898 137.414) (end 200.39 137.922) (width 0.25) (layer F.Cu) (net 2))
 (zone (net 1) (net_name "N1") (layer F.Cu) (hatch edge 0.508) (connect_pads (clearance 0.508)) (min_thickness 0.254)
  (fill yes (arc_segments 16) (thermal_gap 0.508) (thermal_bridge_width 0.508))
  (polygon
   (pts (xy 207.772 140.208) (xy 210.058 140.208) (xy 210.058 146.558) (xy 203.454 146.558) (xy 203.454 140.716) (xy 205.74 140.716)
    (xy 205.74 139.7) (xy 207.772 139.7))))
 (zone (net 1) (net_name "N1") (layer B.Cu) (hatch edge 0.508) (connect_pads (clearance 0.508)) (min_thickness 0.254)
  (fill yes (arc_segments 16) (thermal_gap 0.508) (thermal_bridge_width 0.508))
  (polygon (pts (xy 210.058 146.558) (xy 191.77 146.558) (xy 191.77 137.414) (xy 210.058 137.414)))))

